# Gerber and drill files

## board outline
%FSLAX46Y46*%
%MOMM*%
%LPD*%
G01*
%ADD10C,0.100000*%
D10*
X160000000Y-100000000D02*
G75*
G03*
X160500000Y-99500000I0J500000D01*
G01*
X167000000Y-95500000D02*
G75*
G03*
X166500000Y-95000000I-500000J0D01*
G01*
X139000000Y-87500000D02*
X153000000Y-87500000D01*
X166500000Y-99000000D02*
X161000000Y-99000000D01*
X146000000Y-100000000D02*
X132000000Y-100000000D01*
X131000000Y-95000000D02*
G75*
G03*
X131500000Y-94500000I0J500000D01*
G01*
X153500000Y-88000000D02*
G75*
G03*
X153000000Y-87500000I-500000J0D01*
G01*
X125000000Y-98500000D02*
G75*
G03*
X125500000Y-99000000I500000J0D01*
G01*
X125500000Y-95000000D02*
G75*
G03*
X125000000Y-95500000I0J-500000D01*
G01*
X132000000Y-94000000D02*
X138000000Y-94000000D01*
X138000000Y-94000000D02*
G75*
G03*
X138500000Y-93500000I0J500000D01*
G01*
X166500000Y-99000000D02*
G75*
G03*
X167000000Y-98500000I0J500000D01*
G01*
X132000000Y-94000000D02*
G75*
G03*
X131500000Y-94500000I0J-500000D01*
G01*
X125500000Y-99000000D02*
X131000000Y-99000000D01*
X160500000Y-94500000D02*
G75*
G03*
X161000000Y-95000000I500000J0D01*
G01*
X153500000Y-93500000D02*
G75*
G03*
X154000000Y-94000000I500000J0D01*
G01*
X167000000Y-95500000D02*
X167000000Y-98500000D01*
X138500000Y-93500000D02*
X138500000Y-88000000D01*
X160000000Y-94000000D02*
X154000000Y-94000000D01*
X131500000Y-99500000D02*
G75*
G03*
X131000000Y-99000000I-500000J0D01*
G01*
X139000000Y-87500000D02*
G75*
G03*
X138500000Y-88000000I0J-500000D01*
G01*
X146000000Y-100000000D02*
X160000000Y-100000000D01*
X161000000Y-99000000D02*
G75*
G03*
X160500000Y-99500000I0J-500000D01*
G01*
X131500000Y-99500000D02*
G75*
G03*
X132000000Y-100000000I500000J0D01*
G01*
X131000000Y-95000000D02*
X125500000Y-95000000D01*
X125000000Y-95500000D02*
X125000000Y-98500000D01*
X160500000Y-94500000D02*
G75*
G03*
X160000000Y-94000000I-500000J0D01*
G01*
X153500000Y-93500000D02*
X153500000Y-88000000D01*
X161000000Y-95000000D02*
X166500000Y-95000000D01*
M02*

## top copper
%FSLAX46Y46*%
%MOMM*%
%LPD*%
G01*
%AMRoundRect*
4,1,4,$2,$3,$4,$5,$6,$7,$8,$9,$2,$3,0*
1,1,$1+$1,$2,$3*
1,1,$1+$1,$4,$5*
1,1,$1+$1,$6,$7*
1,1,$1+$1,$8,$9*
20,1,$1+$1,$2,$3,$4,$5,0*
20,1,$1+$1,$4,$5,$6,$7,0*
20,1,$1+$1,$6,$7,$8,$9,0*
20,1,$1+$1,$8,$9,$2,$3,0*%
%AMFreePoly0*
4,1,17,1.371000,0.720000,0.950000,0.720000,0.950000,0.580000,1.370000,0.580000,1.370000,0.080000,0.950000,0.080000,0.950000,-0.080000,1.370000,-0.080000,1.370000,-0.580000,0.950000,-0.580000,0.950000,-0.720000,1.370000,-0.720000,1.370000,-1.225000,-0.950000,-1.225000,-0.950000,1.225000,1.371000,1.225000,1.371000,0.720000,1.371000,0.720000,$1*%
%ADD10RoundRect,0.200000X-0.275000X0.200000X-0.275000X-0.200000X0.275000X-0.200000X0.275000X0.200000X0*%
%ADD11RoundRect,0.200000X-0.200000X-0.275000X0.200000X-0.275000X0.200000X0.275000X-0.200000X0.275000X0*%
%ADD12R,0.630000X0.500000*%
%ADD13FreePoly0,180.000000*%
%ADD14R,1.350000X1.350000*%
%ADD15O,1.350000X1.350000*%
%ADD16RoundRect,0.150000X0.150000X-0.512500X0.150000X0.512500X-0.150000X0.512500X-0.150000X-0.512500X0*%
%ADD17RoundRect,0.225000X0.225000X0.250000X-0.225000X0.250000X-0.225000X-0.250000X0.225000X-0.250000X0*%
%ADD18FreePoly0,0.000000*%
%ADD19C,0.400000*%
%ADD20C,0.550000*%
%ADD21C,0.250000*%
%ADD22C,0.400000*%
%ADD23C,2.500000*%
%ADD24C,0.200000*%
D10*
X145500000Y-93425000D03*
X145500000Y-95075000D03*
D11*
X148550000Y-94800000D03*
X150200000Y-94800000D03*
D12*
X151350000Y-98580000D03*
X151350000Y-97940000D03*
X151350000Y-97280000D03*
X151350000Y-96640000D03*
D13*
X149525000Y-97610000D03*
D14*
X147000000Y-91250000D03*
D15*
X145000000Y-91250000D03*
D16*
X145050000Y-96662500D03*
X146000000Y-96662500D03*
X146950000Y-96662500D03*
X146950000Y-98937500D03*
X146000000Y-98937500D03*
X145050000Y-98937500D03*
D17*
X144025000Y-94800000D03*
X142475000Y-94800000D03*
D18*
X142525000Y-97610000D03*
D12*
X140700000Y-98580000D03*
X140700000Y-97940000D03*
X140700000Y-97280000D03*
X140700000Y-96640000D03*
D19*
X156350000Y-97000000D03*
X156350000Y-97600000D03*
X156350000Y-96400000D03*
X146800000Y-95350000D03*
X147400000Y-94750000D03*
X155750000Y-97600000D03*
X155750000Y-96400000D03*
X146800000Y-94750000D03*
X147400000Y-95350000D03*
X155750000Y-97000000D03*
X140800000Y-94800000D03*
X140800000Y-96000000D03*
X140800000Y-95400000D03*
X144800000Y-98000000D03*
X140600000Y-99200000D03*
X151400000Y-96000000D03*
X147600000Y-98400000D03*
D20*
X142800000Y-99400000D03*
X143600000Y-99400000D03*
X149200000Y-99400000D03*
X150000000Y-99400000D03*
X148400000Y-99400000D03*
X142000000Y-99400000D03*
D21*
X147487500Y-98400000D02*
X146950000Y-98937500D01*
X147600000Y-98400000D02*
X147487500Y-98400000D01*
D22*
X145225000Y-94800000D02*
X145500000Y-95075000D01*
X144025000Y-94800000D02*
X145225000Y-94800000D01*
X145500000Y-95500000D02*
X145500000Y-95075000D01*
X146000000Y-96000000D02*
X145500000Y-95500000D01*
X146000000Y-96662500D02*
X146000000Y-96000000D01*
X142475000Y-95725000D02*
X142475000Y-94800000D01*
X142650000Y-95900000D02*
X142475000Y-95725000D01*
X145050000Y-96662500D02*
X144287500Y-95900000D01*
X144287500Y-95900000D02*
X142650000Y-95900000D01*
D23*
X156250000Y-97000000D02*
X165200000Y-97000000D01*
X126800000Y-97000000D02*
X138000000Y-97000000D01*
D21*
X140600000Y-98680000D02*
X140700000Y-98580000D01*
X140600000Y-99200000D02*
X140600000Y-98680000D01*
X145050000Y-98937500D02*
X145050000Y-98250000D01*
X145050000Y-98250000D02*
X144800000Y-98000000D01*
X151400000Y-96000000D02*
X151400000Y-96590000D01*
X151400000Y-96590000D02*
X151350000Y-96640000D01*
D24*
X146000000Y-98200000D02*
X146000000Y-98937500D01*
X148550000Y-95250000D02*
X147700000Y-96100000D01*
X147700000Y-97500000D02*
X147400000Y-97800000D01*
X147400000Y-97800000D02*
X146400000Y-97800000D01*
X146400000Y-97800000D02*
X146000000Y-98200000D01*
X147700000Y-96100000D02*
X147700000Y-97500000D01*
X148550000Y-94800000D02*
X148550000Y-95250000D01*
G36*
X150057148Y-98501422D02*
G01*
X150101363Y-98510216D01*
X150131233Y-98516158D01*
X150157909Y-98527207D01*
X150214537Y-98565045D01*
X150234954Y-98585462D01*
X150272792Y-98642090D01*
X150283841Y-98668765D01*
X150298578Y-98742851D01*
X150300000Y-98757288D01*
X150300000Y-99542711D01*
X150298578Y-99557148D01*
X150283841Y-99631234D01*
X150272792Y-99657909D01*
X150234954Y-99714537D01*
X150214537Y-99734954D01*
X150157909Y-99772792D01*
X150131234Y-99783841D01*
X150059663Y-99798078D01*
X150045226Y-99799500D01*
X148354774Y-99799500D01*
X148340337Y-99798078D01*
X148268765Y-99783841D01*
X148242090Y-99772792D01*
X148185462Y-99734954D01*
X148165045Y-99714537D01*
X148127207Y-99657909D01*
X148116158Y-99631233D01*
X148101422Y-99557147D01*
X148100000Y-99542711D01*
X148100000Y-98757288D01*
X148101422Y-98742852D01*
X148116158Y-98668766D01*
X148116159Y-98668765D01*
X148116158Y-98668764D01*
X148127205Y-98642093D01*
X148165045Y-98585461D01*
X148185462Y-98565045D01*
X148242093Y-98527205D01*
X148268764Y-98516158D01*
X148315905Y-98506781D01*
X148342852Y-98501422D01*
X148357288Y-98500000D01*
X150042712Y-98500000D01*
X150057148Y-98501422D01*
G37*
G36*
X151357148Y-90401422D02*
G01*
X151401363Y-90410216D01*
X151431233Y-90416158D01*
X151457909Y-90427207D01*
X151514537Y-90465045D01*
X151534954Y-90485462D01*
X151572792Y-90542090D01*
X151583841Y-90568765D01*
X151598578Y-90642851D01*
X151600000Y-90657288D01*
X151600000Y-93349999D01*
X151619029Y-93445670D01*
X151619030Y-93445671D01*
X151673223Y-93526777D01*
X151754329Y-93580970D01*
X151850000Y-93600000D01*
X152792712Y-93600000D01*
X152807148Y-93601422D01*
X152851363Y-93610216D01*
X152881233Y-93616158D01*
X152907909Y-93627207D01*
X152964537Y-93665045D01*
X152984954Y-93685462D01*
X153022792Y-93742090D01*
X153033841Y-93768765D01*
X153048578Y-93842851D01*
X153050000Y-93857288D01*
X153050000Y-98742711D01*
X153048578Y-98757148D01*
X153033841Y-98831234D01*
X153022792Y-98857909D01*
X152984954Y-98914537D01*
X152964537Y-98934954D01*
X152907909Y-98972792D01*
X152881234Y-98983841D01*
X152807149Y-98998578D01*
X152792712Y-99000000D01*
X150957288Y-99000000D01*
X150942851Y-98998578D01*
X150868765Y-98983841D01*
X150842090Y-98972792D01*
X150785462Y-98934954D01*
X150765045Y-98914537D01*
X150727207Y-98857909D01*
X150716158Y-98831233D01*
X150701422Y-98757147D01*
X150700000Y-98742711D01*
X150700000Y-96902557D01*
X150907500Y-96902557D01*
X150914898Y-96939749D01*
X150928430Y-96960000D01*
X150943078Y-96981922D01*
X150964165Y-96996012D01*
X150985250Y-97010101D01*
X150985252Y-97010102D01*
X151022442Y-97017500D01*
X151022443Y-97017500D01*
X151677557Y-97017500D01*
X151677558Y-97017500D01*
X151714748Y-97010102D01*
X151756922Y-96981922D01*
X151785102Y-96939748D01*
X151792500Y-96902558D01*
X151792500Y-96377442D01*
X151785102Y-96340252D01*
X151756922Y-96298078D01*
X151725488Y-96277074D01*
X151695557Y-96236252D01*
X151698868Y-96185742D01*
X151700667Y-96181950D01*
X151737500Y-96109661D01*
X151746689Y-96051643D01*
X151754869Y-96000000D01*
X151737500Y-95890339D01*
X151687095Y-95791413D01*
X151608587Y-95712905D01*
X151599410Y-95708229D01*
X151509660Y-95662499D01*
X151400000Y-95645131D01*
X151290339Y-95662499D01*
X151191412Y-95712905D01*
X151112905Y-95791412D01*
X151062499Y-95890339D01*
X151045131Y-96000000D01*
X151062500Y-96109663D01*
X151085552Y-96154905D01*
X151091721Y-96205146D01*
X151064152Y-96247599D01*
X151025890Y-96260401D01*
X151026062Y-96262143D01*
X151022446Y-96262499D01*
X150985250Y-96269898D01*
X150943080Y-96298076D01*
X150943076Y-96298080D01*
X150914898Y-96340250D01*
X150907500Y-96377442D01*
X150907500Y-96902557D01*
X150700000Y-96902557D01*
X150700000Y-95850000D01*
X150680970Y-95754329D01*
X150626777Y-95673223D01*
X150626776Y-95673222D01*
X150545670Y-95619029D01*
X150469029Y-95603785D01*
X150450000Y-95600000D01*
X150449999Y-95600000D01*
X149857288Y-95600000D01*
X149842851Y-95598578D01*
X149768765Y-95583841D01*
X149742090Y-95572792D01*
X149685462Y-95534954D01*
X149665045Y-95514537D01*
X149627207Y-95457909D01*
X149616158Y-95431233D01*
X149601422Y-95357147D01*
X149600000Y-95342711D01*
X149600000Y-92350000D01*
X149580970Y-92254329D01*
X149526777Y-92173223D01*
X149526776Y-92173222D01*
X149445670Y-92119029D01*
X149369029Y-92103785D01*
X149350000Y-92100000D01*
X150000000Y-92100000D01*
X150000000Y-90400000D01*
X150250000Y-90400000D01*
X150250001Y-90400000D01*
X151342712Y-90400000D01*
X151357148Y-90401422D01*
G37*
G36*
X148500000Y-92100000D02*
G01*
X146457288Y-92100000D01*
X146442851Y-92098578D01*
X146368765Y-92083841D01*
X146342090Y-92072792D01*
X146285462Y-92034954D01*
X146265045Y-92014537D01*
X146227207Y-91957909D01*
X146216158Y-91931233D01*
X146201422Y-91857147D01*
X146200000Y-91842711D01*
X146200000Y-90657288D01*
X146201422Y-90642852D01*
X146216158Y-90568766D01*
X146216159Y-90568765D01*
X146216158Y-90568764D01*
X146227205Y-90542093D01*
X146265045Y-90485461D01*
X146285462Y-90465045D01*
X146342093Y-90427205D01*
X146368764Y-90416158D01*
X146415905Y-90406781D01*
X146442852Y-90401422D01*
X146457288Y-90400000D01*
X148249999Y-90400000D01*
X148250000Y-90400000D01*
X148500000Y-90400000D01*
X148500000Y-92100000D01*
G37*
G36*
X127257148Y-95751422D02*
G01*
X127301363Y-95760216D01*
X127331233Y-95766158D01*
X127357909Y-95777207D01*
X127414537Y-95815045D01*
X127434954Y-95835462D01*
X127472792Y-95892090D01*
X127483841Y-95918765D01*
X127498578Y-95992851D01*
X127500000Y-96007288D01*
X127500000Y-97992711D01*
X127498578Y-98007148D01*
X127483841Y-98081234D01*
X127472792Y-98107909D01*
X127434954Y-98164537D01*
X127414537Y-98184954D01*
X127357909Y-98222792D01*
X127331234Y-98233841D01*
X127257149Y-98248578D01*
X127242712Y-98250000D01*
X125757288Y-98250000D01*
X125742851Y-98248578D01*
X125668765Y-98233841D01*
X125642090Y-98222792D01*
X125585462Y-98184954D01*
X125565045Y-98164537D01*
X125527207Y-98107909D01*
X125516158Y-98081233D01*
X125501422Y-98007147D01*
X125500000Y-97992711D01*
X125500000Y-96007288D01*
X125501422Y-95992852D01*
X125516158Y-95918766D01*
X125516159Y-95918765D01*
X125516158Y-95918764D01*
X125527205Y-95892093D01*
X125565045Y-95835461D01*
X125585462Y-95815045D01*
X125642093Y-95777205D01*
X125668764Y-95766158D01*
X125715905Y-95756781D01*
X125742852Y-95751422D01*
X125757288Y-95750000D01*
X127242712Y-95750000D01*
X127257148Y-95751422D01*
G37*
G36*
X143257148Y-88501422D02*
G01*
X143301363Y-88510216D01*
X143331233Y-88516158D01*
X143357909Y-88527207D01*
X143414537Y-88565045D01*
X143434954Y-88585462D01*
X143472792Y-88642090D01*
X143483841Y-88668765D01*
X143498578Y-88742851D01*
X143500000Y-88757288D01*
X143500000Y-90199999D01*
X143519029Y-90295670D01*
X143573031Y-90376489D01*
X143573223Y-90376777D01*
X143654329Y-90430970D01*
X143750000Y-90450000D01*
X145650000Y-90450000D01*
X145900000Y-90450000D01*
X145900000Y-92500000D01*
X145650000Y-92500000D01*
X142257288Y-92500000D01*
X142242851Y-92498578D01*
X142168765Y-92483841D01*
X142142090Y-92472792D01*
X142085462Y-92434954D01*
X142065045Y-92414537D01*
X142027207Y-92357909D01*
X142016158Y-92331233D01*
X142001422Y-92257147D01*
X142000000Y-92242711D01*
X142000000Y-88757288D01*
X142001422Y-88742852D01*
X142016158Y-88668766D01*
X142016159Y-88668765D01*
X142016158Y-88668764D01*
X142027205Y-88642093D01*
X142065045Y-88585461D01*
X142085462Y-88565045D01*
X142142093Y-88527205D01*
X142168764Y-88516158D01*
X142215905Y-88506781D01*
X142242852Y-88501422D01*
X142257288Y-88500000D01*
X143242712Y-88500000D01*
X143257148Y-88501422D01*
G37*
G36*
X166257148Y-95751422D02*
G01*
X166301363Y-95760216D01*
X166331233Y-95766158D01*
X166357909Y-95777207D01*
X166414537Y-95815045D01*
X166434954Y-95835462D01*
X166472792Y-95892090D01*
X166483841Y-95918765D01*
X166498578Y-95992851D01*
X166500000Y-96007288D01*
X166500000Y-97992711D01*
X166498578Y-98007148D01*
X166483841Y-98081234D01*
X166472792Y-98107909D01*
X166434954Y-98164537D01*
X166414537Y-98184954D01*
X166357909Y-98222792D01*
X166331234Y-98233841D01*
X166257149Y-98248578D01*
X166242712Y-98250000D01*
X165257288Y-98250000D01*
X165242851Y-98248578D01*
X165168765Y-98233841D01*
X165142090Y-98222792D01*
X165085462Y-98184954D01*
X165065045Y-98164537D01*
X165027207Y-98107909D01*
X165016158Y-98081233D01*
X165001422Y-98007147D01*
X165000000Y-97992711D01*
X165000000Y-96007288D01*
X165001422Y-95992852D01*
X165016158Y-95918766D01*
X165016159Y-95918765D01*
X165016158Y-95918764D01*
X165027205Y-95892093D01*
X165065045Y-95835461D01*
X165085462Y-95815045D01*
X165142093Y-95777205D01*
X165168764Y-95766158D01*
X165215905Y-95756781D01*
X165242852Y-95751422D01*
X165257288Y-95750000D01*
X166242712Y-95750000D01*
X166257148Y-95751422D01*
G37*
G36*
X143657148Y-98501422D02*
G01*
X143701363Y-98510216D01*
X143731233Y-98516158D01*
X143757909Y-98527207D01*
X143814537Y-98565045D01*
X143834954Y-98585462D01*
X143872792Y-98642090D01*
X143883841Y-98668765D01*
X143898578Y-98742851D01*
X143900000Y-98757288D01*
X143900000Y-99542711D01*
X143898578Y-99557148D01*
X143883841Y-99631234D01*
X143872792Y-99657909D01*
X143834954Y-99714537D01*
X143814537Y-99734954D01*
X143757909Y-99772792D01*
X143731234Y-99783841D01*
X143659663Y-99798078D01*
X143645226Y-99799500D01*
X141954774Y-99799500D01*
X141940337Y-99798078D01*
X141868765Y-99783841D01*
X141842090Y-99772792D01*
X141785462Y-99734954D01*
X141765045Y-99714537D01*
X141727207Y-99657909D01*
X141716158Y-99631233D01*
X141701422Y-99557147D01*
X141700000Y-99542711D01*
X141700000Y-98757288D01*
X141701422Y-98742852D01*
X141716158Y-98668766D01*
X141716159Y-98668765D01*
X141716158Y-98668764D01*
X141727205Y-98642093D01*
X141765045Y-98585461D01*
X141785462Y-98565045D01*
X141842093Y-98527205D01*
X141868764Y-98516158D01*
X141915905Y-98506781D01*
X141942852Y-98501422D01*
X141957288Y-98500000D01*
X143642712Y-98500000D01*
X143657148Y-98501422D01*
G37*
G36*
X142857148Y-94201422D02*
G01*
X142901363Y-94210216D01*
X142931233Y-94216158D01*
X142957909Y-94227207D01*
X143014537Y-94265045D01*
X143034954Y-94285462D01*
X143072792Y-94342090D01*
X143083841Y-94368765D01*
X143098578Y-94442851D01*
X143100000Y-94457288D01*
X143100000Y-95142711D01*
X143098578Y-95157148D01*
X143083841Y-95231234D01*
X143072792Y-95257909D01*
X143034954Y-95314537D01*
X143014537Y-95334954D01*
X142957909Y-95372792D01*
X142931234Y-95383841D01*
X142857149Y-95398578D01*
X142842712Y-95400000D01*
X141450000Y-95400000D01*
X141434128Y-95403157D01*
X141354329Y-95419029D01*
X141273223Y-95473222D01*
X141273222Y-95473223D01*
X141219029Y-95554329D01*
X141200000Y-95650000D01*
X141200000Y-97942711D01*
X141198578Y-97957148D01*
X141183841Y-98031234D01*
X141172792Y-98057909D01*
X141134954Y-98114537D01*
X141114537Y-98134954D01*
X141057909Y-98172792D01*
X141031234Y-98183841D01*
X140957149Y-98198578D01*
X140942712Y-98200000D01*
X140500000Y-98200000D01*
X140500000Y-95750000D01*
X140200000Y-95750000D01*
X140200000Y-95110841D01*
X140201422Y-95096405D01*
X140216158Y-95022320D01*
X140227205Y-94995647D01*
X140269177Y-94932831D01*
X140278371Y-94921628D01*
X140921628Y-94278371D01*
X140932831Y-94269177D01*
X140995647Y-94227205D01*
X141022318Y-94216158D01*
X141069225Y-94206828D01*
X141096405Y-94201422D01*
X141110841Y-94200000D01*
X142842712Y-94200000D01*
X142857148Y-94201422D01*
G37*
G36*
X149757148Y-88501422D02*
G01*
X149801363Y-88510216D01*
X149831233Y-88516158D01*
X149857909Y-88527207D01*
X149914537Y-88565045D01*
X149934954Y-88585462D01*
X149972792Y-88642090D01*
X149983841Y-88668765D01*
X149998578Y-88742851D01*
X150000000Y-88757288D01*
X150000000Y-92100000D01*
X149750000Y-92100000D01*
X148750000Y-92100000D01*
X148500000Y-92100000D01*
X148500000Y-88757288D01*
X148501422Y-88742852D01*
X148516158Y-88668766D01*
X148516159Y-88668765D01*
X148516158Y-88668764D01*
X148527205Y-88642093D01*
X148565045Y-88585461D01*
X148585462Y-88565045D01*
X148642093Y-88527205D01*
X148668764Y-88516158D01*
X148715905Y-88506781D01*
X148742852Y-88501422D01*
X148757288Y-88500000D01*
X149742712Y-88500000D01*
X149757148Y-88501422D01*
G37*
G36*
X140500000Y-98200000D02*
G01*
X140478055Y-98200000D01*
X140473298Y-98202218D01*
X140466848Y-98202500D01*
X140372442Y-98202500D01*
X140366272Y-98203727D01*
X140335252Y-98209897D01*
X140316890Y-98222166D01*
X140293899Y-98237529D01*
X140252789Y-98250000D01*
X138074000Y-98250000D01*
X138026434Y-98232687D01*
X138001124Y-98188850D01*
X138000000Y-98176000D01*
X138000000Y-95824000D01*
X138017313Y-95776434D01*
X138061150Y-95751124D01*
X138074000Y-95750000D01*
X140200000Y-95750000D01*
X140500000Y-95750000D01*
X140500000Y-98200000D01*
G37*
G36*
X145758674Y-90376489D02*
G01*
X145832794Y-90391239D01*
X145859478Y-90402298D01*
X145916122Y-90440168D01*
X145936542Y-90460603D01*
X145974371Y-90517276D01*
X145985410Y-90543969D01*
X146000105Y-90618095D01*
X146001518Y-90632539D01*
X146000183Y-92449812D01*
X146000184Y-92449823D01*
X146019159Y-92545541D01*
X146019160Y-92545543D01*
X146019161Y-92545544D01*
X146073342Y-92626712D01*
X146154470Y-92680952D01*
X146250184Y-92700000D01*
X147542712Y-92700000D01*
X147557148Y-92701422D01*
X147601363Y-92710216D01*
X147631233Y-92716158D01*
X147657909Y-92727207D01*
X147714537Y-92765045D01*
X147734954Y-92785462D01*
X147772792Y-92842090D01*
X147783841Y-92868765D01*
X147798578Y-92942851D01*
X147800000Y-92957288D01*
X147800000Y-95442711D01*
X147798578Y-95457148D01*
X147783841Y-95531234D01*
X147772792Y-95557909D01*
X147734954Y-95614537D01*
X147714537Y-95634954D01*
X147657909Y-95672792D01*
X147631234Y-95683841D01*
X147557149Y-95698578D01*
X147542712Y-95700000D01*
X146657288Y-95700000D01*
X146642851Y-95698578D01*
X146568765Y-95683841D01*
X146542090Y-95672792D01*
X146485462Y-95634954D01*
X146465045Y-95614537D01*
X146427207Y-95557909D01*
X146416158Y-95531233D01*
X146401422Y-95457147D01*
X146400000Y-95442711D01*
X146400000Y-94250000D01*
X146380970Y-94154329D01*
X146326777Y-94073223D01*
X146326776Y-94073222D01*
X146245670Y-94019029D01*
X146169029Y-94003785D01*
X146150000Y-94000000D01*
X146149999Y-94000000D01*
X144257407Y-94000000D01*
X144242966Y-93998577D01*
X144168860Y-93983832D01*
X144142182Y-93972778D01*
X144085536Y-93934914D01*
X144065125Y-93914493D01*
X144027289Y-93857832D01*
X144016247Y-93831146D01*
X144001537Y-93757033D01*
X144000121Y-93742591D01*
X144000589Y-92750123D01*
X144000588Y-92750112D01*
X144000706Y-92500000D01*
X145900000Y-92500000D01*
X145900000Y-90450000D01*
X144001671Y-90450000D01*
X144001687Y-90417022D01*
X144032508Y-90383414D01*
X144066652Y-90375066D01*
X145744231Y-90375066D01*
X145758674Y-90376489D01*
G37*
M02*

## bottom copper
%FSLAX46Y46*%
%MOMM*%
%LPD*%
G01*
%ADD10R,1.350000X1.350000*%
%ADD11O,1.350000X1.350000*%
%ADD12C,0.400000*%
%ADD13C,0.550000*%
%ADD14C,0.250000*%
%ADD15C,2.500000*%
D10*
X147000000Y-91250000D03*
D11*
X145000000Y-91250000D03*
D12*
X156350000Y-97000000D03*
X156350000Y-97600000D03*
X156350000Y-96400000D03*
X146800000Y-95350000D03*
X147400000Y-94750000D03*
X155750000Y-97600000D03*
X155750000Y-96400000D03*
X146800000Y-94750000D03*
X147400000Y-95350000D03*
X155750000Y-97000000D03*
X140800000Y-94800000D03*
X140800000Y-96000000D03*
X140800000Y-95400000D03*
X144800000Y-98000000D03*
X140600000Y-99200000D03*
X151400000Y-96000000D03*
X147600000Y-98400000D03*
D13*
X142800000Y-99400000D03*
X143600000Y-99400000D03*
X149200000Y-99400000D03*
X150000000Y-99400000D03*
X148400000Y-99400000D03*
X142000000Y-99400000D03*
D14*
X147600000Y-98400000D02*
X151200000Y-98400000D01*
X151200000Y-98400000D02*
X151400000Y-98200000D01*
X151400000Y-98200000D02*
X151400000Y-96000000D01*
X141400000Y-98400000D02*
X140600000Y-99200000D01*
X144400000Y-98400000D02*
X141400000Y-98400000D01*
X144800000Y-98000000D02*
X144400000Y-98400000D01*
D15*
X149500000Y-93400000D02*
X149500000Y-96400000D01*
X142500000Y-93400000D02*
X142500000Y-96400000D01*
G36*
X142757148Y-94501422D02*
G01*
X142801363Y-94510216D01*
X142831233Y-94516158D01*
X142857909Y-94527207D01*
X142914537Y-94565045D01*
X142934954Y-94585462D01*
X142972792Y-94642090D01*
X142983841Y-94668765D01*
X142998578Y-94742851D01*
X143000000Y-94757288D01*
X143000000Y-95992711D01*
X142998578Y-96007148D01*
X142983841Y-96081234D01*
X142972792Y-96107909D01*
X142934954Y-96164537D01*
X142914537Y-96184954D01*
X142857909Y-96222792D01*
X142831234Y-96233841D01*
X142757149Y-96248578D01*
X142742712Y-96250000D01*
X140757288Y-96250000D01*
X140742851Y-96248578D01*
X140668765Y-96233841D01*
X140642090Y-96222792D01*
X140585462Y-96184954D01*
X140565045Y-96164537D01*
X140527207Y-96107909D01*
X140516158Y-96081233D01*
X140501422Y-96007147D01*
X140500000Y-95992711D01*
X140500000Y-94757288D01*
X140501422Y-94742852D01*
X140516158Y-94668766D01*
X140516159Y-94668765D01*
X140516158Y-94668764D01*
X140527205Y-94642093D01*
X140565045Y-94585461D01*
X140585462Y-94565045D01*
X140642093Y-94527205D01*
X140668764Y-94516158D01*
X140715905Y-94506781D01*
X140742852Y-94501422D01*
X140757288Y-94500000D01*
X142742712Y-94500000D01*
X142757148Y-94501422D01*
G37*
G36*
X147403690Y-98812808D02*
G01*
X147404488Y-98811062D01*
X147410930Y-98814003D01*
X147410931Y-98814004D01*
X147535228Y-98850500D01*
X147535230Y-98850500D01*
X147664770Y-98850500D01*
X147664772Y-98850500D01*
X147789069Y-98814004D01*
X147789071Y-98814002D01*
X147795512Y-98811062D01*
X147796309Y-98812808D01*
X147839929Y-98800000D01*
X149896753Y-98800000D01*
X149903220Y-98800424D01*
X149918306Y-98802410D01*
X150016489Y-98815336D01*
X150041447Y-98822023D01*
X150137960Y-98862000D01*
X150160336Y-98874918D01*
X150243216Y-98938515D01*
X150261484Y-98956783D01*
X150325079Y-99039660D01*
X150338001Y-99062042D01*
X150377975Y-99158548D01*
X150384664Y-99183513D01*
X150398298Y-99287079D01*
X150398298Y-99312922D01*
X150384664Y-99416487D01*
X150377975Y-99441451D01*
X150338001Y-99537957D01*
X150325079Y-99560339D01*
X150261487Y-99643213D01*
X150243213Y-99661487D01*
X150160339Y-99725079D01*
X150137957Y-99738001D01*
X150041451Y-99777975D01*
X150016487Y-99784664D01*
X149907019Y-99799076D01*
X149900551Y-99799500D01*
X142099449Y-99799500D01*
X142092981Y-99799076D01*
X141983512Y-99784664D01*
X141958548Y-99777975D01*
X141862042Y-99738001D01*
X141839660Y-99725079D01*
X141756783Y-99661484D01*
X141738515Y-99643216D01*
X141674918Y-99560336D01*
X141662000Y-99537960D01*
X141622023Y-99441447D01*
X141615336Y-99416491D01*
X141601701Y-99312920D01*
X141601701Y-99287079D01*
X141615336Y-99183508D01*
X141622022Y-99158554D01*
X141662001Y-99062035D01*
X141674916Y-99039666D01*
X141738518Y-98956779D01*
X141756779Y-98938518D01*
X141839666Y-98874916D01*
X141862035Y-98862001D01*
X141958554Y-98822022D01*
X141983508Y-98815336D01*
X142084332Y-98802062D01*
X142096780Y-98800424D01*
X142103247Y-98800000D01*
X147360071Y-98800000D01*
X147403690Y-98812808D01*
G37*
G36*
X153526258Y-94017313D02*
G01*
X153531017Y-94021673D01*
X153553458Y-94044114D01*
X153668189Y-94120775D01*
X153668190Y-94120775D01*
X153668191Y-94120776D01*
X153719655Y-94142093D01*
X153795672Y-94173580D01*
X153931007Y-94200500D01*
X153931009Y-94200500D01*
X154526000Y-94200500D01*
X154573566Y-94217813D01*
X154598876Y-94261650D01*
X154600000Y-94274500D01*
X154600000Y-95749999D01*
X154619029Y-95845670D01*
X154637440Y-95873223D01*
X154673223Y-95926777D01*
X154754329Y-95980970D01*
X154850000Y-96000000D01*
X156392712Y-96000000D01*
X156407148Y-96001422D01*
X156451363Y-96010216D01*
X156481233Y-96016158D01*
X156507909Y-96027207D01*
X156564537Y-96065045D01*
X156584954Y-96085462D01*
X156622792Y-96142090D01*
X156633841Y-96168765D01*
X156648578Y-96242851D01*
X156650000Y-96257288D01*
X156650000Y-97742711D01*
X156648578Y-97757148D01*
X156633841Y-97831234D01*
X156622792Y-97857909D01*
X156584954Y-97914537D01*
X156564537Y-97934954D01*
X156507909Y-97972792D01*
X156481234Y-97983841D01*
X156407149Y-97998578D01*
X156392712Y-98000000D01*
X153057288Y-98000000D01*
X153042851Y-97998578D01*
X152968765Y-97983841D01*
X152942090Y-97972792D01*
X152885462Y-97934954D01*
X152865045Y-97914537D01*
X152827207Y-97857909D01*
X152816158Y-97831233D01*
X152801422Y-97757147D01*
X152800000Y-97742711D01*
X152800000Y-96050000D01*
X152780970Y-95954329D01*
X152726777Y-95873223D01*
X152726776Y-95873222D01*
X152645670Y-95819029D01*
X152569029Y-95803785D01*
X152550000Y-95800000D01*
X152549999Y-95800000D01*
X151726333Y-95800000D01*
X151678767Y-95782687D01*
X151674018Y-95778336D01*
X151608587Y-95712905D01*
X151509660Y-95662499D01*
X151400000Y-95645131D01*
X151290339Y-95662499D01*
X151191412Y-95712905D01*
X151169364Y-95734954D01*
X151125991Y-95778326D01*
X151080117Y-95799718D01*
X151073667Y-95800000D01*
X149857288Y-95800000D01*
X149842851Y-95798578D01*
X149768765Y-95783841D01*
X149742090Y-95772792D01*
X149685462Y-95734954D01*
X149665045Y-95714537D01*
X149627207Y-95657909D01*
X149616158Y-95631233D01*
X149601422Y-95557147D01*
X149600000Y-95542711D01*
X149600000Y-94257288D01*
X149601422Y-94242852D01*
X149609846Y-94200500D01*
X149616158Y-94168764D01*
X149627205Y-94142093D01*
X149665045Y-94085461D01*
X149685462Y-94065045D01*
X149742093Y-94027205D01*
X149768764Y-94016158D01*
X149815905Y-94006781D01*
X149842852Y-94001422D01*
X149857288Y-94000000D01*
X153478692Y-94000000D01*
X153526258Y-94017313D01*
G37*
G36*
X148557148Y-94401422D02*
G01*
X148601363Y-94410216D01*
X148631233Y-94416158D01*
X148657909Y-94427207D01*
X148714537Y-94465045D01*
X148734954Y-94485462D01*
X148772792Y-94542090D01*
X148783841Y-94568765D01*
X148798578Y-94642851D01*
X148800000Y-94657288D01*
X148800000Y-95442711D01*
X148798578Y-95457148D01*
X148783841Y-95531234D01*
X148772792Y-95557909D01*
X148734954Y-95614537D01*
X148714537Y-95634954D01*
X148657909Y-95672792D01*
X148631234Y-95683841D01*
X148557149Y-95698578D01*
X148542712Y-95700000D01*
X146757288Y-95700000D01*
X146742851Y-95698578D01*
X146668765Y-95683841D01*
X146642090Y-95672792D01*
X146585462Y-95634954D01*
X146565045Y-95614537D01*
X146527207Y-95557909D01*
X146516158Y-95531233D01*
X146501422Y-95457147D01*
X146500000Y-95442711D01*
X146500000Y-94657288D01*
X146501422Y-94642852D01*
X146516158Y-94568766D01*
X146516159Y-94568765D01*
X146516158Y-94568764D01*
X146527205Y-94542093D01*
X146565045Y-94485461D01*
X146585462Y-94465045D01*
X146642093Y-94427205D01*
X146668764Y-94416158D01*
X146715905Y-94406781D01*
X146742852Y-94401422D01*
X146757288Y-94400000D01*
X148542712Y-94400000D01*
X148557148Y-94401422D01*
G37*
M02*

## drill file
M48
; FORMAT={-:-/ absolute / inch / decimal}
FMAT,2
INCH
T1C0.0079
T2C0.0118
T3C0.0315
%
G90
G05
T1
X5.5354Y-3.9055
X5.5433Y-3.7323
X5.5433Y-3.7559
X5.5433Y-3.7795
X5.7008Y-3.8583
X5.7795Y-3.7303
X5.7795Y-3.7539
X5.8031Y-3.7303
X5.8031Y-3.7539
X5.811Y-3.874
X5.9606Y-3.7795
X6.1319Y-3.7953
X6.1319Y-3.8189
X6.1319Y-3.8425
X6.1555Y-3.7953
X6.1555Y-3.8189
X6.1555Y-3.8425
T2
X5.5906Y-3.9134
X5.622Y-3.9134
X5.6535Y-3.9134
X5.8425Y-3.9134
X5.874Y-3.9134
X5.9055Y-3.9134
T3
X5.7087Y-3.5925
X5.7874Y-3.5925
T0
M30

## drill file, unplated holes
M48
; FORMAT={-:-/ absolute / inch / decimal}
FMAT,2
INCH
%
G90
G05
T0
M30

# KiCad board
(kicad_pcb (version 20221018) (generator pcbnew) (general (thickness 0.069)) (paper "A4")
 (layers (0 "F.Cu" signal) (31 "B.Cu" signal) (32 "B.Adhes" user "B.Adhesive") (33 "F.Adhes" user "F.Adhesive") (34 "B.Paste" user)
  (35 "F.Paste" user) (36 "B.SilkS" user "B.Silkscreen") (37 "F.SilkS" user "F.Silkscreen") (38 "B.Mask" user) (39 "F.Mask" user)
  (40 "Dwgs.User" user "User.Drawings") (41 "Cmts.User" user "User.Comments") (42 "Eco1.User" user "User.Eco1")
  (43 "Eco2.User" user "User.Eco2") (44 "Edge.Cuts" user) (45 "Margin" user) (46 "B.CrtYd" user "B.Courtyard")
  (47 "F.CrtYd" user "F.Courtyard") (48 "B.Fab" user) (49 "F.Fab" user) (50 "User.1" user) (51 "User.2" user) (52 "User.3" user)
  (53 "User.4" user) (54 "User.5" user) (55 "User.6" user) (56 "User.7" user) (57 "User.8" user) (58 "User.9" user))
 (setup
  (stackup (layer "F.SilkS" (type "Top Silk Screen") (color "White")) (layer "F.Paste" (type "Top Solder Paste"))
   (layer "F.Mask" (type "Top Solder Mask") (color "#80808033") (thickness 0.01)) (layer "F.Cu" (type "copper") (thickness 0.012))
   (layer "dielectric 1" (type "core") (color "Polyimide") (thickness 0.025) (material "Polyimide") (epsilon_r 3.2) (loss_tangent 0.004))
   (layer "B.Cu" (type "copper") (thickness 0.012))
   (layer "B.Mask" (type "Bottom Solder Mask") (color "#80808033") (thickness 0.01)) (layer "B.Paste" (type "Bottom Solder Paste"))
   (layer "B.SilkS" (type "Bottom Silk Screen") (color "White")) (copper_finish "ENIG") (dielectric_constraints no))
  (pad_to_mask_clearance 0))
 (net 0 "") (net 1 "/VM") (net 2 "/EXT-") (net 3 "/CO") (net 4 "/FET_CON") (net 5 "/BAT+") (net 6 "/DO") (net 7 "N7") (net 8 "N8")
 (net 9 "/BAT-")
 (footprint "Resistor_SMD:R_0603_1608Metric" (layer "F.Cu") (at 149.375 94.8)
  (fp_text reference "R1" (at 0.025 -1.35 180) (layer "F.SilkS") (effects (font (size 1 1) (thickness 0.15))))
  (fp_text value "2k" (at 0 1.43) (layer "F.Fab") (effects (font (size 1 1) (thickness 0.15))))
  (pad "1" smd roundrect (at -0.825 0) (size 0.8 0.95) (layers "F.Cu" "F.Paste" "F.Mask") (roundrect_rratio 0.25) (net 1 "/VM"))
  (pad "2" smd roundrect (at 0.825 0) (size 0.8 0.95) (layers "F.Cu" "F.Paste" "F.Mask") (roundrect_rratio 0.25) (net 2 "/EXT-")))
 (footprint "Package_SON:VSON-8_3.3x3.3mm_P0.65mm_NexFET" (layer "F.Cu") (at 149.91 97.61 180)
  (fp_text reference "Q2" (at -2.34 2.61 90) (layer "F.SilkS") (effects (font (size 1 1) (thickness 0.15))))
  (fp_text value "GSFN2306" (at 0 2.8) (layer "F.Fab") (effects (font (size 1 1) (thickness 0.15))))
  (pad "" smd rect (at -0.09 -0.61 180) (size 0.57 0.738) (layers "F.Paste"))
  (pad "" smd rect (at -0.09 0.61 180) (size 0.57 0.738) (layers "F.Paste"))
  (pad "" smd rect (at 0.86 -0.61 180) (size 0.57 0.738) (layers "F.Paste"))
  (pad "" smd rect (at 0.86 0.61 180) (size 0.57 0.738) (layers "F.Paste"))
  (pad "" smd rect (at 1.44 -0.9725 180) (size 0.63 0.505) (layers "F.Paste"))
  (pad "" smd rect (at 1.44 -0.33 180) (size 0.63 0.5) (layers "F.Paste"))
  (pad "" smd rect (at 1.44 0.33 180) (size 0.63 0.5) (layers "F.Paste"))
  (pad "" smd rect (at 1.44 0.9725 180) (size 0.63 0.505) (layers "F.Paste"))
  (pad "1" smd rect (at -1.44 -0.97 180) (size 0.63 0.5) (layers "F.Cu" "F.Paste" "F.Mask") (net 2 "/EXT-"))
  (pad "2" smd rect (at -1.44 -0.33 180) (size 0.63 0.5) (layers "F.Cu" "F.Paste" "F.Mask") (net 2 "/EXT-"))
  (pad "3" smd rect (at -1.44 0.33 180) (size 0.63 0.5) (layers "F.Cu" "F.Paste" "F.Mask") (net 2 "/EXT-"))
  (pad "4" smd rect (at -1.44 0.97 180) (size 0.63 0.5) (layers "F.Cu" "F.Paste" "F.Mask") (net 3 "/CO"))
  (pad "5" smd custom (at 0.385 0 180) (size 1.9 2.45) (layers "F.Cu" "F.Mask") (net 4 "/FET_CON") (thermal_bridge_angle 45)
   (options (clearance outline) (anchor rect)) (primitives)))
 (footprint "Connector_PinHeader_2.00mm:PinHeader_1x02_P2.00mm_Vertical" (layer "F.Cu") (at 147 91.25 -90)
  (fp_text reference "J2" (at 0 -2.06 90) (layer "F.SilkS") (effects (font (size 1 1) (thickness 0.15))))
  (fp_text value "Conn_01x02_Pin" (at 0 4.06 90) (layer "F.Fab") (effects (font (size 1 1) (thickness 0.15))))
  (pad "1" thru_hole rect (at 0 0 270) (size 1.35 1.35) (drill 0.8) (layers "*.Cu" "*.Mask") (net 2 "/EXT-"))
  (pad "2" thru_hole oval (at 0 2 270) (size 1.35 1.35) (drill 0.8) (layers "*.Cu" "*.Mask") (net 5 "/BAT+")))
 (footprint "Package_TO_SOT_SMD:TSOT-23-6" (layer "F.Cu") (at 146 97.8 90)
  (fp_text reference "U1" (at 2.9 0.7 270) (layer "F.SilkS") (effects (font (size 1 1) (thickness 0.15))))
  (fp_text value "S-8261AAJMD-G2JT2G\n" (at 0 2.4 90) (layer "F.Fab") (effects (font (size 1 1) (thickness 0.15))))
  (pad "1" smd roundrect (at -1.1375 -0.95 90) (size 1.325 0.6) (layers "F.Cu" "F.Paste" "F.Mask") (roundrect_rratio 0.25) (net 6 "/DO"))
  (pad "2" smd roundrect (at -1.1375 0 90) (size 1.325 0.6) (layers "F.Cu" "F.Paste" "F.Mask") (roundrect_rratio 0.25) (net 1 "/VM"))
  (pad "3" smd roundrect (at -1.1375 0.95 90) (size 1.325 0.6) (layers "F.Cu" "F.Paste" "F.Mask") (roundrect_rratio 0.25) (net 3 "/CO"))
  (pad "4" smd roundrect (at 1.1375 0.95 90) (size 1.325 0.6) (layers "F.Cu" "F.Paste" "F.Mask") (roundrect_rratio 0.25) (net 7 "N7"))
  (pad "5" smd roundrect (at 1.1375 0 90) (size 1.325 0.6) (layers "F.Cu" "F.Paste" "F.Mask") (roundrect_rratio 0.25) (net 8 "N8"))
  (pad "6" smd roundrect (at 1.1375 -0.95 90) (size 1.325 0.6) (layers "F.Cu" "F.Paste" "F.Mask") (roundrect_rratio 0.25) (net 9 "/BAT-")))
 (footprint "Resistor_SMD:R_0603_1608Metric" (layer "F.Cu") (at 145.5 94.25 -90)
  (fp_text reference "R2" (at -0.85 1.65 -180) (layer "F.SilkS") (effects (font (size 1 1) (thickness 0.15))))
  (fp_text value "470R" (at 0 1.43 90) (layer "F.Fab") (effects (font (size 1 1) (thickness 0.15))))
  (pad "1" smd roundrect (at -0.825 0 270) (size 0.8 0.95) (layers "F.Cu" "F.Paste" "F.Mask") (roundrect_rratio 0.25) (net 5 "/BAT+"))
  (pad "2" smd roundrect (at 0.825 0 270) (size 0.8 0.95) (layers "F.Cu" "F.Paste" "F.Mask") (roundrect_rratio 0.25) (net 8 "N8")))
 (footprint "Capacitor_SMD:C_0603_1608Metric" (layer "F.Cu") (at 143.25 94.8 180)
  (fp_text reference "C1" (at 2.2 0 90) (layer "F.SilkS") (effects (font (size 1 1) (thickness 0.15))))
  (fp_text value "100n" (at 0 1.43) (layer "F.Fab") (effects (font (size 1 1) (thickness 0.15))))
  (pad "1" smd roundrect (at -0.775 0 180) (size 0.9 0.95) (layers "F.Cu" "F.Paste" "F.Mask") (roundrect_rratio 0.25) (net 8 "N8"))
  (pad "2" smd roundrect (at 0.775 0 180) (size 0.9 0.95) (layers "F.Cu" "F.Paste" "F.Mask") (roundrect_rratio 0.25) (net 9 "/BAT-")))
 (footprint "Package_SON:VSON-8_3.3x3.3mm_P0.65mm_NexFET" (layer "F.Cu") (at 142.14 97.61)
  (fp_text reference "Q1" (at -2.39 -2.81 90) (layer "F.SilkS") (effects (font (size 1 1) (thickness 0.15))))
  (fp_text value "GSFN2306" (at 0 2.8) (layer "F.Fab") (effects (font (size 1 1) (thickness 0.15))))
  (pad "" smd rect (at -0.09 -0.61) (size 0.57 0.738) (layers "F.Paste"))
  (pad "" smd rect (at -0.09 0.61) (size 0.57 0.738) (layers "F.Paste"))
  (pad "" smd rect (at 0.86 -0.61) (size 0.57 0.738) (layers "F.Paste"))
  (pad "" smd rect (at 0.86 0.61) (size 0.57 0.738) (layers "F.Paste"))
  (pad "" smd rect (at 1.44 -0.9725) (size 0.63 0.505) (layers "F.Paste"))
  (pad "" smd rect (at 1.44 -0.33) (size 0.63 0.5) (layers "F.Paste"))
  (pad "" smd rect (at 1.44 0.33) (size 0.63 0.5) (layers "F.Paste"))
  (pad "" smd rect (at 1.44 0.9725) (size 0.63 0.505) (layers "F.Paste"))
  (pad "1" smd rect (at -1.44 -0.97) (size 0.63 0.5) (layers "F.Cu" "F.Paste" "F.Mask") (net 9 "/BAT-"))
  (pad "2" smd rect (at -1.44 -0.33) (size 0.63 0.5) (layers "F.Cu" "F.Paste" "F.Mask") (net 9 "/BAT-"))
  (pad "3" smd rect (at -1.44 0.33) (size 0.63 0.5) (layers "F.Cu" "F.Paste" "F.Mask") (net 9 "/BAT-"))
  (pad "4" smd rect (at -1.44 0.97) (size 0.63 0.5) (layers "F.Cu" "F.Paste" "F.Mask") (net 6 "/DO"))
  (pad "5" smd custom (at 0.385 0) (size 1.9 2.45) (layers "F.Cu" "F.Mask") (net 4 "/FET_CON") (thermal_bridge_angle 45)
   (options (clearance outline) (anchor rect)) (primitives)))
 (gr_arc (start 160.5 99.5) (mid 160.353553 99.853553) (end 160 100) (stroke (width 0.1) (type default)) (layer "Edge.Cuts"))
 (gr_arc (start 166.5 95) (mid 166.853553 95.146447) (end 167 95.5) (stroke (width 0.1) (type default)) (layer "Edge.Cuts"))
 (gr_line (start 139 87.5) (end 153 87.5) (stroke (width 0.1) (type default)) (layer "Edge.Cuts"))
 (gr_line (start 166.5 99) (end 161 99) (stroke (width 0.1) (type default)) (layer "Edge.Cuts"))
 (gr_line (start 146 100) (end 132 100) (stroke (width 0.1) (type default)) (layer "Edge.Cuts"))
 (gr_arc (start 131.5 94.5) (mid 131.353553 94.853553) (end 131 95) (stroke (width 0.1) (type default)) (layer "Edge.Cuts"))
 (gr_arc (start 153 87.5) (mid 153.353553 87.646447) (end 153.5 88) (stroke (width 0.1) (type default)) (layer "Edge.Cuts"))
 (gr_arc (start 125.5 99) (mid 125.146447 98.853553) (end 125 98.5) (stroke (width 0.1) (type default)) (layer "Edge.Cuts"))
 (gr_arc (start 125 95.5) (mid 125.146447 95.146447) (end 125.5 95) (stroke (width 0.1) (type default)) (layer "Edge.Cuts"))
 (gr_line (start 132 94) (end 138 94) (stroke (width 0.1) (type default)) (layer "Edge.Cuts"))
 (gr_arc (start 138.5 93.5) (mid 138.353553 93.853553) (end 138 94) (stroke (width 0.1) (type default)) (layer "Edge.Cuts"))
 (gr_arc (start 167 98.5) (mid 166.853553 98.853553) (end 166.5 99) (stroke (width 0.1) (type default)) (layer "Edge.Cuts"))
 (gr_arc (start 131.5 94.5) (mid 131.646447 94.146447) (end 132 94) (stroke (width 0.1) (type default)) (layer "Edge.Cuts"))
 (gr_line (start 125.5 99) (end 131 99) (stroke (width 0.1) (type default)) (layer "Edge.Cuts"))
 (gr_arc (start 161 95) (mid 160.646447 94.853553) (end 160.5 94.5) (stroke (width 0.1) (type default)) (layer "Edge.Cuts"))
 (gr_arc (start 154 94) (mid 153.646447 93.853553) (end 153.5 93.5) (stroke (width 0.1) (type default)) (layer "Edge.Cuts"))
 (gr_line (start 167 95.5) (end 167 98.5) (stroke (width 0.1) (type default)) (layer "Edge.Cuts"))
 (gr_line (start 138.5 93.5) (end 138.5 88) (stroke (width 0.1) (type default)) (layer "Edge.Cuts"))
 (gr_line (start 160 94) (end 154 94) (stroke (width 0.1) (type default)) (layer "Edge.Cuts"))
 (gr_arc (start 131 99) (mid 131.353553 99.146447) (end 131.5 99.5) (stroke (width 0.1) (type default)) (layer "Edge.Cuts"))
 (gr_arc (start 138.5 88) (mid 138.646447 87.646447) (end 139 87.5) (stroke (width 0.1) (type default)) (layer "Edge.Cuts"))
 (gr_line (start 146 100) (end 160 100) (stroke (width 0.1) (type default)) (layer "Edge.Cuts"))
 (gr_arc (start 160.5 99.5) (mid 160.646447 99.146447) (end 161 99) (stroke (width 0.1) (type default)) (layer "Edge.Cuts"))
 (gr_arc (start 132 100) (mid 131.646447 99.853553) (end 131.5 99.5) (stroke (width 0.1) (type default)) (layer "Edge.Cuts"))
 (gr_line (start 131 95) (end 125.5 95) (stroke (width 0.1) (type default)) (layer "Edge.Cuts"))
 (gr_line (start 125 95.5) (end 125 98.5) (stroke (width 0.1) (type default)) (layer "Edge.Cuts"))
 (gr_arc (start 160 94) (mid 160.353553 94.146447) (end 160.5 94.5) (stroke (width 0.1) (type default)) (layer "Edge.Cuts"))
 (gr_line (start 153.5 93.5) (end 153.5 88) (stroke (width 0.1) (type default)) (layer "Edge.Cuts"))
 (gr_line (start 161 95) (end 166.5 95) (stroke (width 0.1) (type default)) (layer "Edge.Cuts"))
 (segment (start 156.25 97) (end 165.2 97) (width 2.5) (layer "F.Cu") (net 5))
 (via (at 156.35 97) (size 0.4) (drill 0.2) (layers "F.Cu" "B.Cu") (free) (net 5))
 (via (at 156.35 97.6) (size 0.4) (drill 0.2) (layers "F.Cu" "B.Cu") (free) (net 5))
 (via (at 156.35 96.4) (size 0.4) (drill 0.2) (layers "F.Cu" "B.Cu") (free) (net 5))
 (via (at 146.8 95.35) (size 0.4) (drill 0.2) (layers "F.Cu" "B.Cu") (free) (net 5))
 (via (at 147.4 94.75) (size 0.4) (drill 0.2) (layers "F.Cu" "B.Cu") (free) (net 5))
 (via (at 155.75 97.6) (size 0.4) (drill 0.2) (layers "F.Cu" "B.Cu") (free) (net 5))
 (via (at 155.75 96.4) (size 0.4) (drill 0.2) (layers "F.Cu" "B.Cu") (free) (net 5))
 (via (at 146.8 94.75) (size 0.4) (drill 0.2) (layers "F.Cu" "B.Cu") (free) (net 5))
 (via (at 147.4 95.35) (size 0.4) (drill 0.2) (layers "F.Cu" "B.Cu") (free) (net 5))
 (via (at 155.75 97) (size 0.4) (drill 0.2) (layers "F.Cu" "B.Cu") (free) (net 5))
 (segment (start 149.5 93.4) (end 149.5 96.4) (width 2.5) (layer "B.Cu") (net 5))
 (segment (start 142.475 95.725) (end 142.475 94.8) (width 0.4) (layer "F.Cu") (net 9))
 (segment (start 144.2875 95.9) (end 142.65 95.9) (width 0.4) (layer "F.Cu") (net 9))
 (segment (start 145.05 96.6625) (end 144.2875 95.9) (width 0.4) (layer "F.Cu") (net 9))
 (segment (start 142.65 95.9) (end 142.475 95.725) (width 0.4) (layer "F.Cu") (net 9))
 (segment (start 126.8 97) (end 138 97) (width 2.5) (layer "F.Cu") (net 9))
 (via (at 140.8 94.8) (size 0.4) (drill 0.2) (layers "F.Cu" "B.Cu") (free) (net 9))
 (via (at 140.8 96) (size 0.4) (drill 0.2) (layers "F.Cu" "B.Cu") (free) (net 9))
 (via (at 140.8 95.4) (size 0.4) (drill 0.2) (layers "F.Cu" "B.Cu") (free) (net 9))
 (segment (start 142.5 93.4) (end 142.5 96.4) (width 2.5) (layer "B.Cu") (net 9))
 (segment (start 140.6 98.68) (end 140.7 98.58) (width 0.25) (layer "F.Cu") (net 6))
 (segment (start 140.6 99.2) (end 140.6 98.68) (width 0.25) (layer "F.Cu") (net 6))
 (segment (start 145.05 98.9375) (end 145.05 98.25) (width 0.25) (layer "F.Cu") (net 6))
 (segment (start 145.05 98.25) (end 144.8 98) (width 0.25) (layer "F.Cu") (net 6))
 (via (at 144.8 98) (size 0.4) (drill 0.2) (layers "F.Cu" "B.Cu") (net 6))
 (via (at 140.6 99.2) (size 0.4) (drill 0.2) (layers "F.Cu" "B.Cu") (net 6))
 (segment (start 144.8 98) (end 144.4 98.4) (width 0.25) (layer "B.Cu") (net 6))
 (segment (start 144.4 98.4) (end 141.4 98.4) (width 0.25) (layer "B.Cu") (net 6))
 (segment (start 141.4 98.4) (end 140.6 99.2) (width 0.25) (layer "B.Cu") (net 6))
 (segment (start 151.4 96) (end 151.4 96.59) (width 0.25) (layer "F.Cu") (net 3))
 (segment (start 147.6 98.4) (end 147.4875 98.4) (width 0.25) (layer "F.Cu") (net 3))
 (segment (start 147.4875 98.4) (end 146.95 98.9375) (width 0.25) (layer "F.Cu") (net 3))
 (segment (start 151.4 96.59) (end 151.35 96.64) (width 0.25) (layer "F.Cu") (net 3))
 (via (at 151.4 96) (size 0.4) (drill 0.2) (layers "F.Cu" "B.Cu") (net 3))
 (via (at 147.6 98.4) (size 0.4) (drill 0.2) (layers "F.Cu" "B.Cu") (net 3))
 (segment (start 147.6 98.4) (end 151.2 98.4) (width 0.25) (layer "B.Cu") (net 3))
 (segment (start 151.2 98.4) (end 151.4 98.2) (width 0.25) (layer "B.Cu") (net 3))
 (segment (start 151.4 98.2) (end 151.4 96) (width 0.25) (layer "B.Cu") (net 3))
 (segment (start 146 98.2) (end 146 98.9375) (width 0.2) (layer "F.Cu") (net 1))
 (segment (start 148.55 95.25) (end 147.7 96.1) (width 0.2) (layer "F.Cu") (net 1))
 (segment (start 147.7 97.5) (end 147.4 97.8) (width 0.2) (layer "F.Cu") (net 1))
 (segment (start 147.4 97.8) (end 146.4 97.8) (width 0.2) (layer "F.Cu") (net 1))
 (segment (start 146.4 97.8) (end 146 98.2) (width 0.2) (layer "F.Cu") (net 1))
 (segment (start 147.7 96.1) (end 147.7 97.5) (width 0.2) (layer "F.Cu") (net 1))
 (segment (start 148.55 94.8) (end 148.55 95.25) (width 0.2) (layer "F.Cu") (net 1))
 (via (at 142.8 99.4) (size 0.55) (drill 0.3) (layers "F.Cu" "B.Cu") (free) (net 4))
 (via (at 143.6 99.4) (size 0.55) (drill 0.3) (layers "F.Cu" "B.Cu") (free) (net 4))
 (via (at 149.2 99.4) (size 0.55) (drill 0.3) (layers "F.Cu" "B.Cu") (free) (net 4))
 (via (at 150 99.4) (size 0.55) (drill 0.3) (layers "F.Cu" "B.Cu") (free) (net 4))
 (via (at 148.4 99.4) (size 0.55) (drill 0.3) (layers "F.Cu" "B.Cu") (free) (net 4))
 (via (at 142 99.4) (size 0.55) (drill 0.3) (layers "F.Cu" "B.Cu") (free) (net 4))
 (segment (start 146 96.6625) (end 146 96) (width 0.4) (layer "F.Cu") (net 8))
 (segment (start 144.025 94.8) (end 145.225 94.8) (width 0.4) (layer "F.Cu") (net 8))
 (segment (start 146 96) (end 145.5 95.5) (width 0.4) (layer "F.Cu") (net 8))
 (segment (start 145.5 95.5) (end 145.5 95.075) (width 0.4) (layer "F.Cu") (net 8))
 (segment (start 145.225 94.8) (end 145.5 95.075) (width 0.4) (layer "F.Cu") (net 8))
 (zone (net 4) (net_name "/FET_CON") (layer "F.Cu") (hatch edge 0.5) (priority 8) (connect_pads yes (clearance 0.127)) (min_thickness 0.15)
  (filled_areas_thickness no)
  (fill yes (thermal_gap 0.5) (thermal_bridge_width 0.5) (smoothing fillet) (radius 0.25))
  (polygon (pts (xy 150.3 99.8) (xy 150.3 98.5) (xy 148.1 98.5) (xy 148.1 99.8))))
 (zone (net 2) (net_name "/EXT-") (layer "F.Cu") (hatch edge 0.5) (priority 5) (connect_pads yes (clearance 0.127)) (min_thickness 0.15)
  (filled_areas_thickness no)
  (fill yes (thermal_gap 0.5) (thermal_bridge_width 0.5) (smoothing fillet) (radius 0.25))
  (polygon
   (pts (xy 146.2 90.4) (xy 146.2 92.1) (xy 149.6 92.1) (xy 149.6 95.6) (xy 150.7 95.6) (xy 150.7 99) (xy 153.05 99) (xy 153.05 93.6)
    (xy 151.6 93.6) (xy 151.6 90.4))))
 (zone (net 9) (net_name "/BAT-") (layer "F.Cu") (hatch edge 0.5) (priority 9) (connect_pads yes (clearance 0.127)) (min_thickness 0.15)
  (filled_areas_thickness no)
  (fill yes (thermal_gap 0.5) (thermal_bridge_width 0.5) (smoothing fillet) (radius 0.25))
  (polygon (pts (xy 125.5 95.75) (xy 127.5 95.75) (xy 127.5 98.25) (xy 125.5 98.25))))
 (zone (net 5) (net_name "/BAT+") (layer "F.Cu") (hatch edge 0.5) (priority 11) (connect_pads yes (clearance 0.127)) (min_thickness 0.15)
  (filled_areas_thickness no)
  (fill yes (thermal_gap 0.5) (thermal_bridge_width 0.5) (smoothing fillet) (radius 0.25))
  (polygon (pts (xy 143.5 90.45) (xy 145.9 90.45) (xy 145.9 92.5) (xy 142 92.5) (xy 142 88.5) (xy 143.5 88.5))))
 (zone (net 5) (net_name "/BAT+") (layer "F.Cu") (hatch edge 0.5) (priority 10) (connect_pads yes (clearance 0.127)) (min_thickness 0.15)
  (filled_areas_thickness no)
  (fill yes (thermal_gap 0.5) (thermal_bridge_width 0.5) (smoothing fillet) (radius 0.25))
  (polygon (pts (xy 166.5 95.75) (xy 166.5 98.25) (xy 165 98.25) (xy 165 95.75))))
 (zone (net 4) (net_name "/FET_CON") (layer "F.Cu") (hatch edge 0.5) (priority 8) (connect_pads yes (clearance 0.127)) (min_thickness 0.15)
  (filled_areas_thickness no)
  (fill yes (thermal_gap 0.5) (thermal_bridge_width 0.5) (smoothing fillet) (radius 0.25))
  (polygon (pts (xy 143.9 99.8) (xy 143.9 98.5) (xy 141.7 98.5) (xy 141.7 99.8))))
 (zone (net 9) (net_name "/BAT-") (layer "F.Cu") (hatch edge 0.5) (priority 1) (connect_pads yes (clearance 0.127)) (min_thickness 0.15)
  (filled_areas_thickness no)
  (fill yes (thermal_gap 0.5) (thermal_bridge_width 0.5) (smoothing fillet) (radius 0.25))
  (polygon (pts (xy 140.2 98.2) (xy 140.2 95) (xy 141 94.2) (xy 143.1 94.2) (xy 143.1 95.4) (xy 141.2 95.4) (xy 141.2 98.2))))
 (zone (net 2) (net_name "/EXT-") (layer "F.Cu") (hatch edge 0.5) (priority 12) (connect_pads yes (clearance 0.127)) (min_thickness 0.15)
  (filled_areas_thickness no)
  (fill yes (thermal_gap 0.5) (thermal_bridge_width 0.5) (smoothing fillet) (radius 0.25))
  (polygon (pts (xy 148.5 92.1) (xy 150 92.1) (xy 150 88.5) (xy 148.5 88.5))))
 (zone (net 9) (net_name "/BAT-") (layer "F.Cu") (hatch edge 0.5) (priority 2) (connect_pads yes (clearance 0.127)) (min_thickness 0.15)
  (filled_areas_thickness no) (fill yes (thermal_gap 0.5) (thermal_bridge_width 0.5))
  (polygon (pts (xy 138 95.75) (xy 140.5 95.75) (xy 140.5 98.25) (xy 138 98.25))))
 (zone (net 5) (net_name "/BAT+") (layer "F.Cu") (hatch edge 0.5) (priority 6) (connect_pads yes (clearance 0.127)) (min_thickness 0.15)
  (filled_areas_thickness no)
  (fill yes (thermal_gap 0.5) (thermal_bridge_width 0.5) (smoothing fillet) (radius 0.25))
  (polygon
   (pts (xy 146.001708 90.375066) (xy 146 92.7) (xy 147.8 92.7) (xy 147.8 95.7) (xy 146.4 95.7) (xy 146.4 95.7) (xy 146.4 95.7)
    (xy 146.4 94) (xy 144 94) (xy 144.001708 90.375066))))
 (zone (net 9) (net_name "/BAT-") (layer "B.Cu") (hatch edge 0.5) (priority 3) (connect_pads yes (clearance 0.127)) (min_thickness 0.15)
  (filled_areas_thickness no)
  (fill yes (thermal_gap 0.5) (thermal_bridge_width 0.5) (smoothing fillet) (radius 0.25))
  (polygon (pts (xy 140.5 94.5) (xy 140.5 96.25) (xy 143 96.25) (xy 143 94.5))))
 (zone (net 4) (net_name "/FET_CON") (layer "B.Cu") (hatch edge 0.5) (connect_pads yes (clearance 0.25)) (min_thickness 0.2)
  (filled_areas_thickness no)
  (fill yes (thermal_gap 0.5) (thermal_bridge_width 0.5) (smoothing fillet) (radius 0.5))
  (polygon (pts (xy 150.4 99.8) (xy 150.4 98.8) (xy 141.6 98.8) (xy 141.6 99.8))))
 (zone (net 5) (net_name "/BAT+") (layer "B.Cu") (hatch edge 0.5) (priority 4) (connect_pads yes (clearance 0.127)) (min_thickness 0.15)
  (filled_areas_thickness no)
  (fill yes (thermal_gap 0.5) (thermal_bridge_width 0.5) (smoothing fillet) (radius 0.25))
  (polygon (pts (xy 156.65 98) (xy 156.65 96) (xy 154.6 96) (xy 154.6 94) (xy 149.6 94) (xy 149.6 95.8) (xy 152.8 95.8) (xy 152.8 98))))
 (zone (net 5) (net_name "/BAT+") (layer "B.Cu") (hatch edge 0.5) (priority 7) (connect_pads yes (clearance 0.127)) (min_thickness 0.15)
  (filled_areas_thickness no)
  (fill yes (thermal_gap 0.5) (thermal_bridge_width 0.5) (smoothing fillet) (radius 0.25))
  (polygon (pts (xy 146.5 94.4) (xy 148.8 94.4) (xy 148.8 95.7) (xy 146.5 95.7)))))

